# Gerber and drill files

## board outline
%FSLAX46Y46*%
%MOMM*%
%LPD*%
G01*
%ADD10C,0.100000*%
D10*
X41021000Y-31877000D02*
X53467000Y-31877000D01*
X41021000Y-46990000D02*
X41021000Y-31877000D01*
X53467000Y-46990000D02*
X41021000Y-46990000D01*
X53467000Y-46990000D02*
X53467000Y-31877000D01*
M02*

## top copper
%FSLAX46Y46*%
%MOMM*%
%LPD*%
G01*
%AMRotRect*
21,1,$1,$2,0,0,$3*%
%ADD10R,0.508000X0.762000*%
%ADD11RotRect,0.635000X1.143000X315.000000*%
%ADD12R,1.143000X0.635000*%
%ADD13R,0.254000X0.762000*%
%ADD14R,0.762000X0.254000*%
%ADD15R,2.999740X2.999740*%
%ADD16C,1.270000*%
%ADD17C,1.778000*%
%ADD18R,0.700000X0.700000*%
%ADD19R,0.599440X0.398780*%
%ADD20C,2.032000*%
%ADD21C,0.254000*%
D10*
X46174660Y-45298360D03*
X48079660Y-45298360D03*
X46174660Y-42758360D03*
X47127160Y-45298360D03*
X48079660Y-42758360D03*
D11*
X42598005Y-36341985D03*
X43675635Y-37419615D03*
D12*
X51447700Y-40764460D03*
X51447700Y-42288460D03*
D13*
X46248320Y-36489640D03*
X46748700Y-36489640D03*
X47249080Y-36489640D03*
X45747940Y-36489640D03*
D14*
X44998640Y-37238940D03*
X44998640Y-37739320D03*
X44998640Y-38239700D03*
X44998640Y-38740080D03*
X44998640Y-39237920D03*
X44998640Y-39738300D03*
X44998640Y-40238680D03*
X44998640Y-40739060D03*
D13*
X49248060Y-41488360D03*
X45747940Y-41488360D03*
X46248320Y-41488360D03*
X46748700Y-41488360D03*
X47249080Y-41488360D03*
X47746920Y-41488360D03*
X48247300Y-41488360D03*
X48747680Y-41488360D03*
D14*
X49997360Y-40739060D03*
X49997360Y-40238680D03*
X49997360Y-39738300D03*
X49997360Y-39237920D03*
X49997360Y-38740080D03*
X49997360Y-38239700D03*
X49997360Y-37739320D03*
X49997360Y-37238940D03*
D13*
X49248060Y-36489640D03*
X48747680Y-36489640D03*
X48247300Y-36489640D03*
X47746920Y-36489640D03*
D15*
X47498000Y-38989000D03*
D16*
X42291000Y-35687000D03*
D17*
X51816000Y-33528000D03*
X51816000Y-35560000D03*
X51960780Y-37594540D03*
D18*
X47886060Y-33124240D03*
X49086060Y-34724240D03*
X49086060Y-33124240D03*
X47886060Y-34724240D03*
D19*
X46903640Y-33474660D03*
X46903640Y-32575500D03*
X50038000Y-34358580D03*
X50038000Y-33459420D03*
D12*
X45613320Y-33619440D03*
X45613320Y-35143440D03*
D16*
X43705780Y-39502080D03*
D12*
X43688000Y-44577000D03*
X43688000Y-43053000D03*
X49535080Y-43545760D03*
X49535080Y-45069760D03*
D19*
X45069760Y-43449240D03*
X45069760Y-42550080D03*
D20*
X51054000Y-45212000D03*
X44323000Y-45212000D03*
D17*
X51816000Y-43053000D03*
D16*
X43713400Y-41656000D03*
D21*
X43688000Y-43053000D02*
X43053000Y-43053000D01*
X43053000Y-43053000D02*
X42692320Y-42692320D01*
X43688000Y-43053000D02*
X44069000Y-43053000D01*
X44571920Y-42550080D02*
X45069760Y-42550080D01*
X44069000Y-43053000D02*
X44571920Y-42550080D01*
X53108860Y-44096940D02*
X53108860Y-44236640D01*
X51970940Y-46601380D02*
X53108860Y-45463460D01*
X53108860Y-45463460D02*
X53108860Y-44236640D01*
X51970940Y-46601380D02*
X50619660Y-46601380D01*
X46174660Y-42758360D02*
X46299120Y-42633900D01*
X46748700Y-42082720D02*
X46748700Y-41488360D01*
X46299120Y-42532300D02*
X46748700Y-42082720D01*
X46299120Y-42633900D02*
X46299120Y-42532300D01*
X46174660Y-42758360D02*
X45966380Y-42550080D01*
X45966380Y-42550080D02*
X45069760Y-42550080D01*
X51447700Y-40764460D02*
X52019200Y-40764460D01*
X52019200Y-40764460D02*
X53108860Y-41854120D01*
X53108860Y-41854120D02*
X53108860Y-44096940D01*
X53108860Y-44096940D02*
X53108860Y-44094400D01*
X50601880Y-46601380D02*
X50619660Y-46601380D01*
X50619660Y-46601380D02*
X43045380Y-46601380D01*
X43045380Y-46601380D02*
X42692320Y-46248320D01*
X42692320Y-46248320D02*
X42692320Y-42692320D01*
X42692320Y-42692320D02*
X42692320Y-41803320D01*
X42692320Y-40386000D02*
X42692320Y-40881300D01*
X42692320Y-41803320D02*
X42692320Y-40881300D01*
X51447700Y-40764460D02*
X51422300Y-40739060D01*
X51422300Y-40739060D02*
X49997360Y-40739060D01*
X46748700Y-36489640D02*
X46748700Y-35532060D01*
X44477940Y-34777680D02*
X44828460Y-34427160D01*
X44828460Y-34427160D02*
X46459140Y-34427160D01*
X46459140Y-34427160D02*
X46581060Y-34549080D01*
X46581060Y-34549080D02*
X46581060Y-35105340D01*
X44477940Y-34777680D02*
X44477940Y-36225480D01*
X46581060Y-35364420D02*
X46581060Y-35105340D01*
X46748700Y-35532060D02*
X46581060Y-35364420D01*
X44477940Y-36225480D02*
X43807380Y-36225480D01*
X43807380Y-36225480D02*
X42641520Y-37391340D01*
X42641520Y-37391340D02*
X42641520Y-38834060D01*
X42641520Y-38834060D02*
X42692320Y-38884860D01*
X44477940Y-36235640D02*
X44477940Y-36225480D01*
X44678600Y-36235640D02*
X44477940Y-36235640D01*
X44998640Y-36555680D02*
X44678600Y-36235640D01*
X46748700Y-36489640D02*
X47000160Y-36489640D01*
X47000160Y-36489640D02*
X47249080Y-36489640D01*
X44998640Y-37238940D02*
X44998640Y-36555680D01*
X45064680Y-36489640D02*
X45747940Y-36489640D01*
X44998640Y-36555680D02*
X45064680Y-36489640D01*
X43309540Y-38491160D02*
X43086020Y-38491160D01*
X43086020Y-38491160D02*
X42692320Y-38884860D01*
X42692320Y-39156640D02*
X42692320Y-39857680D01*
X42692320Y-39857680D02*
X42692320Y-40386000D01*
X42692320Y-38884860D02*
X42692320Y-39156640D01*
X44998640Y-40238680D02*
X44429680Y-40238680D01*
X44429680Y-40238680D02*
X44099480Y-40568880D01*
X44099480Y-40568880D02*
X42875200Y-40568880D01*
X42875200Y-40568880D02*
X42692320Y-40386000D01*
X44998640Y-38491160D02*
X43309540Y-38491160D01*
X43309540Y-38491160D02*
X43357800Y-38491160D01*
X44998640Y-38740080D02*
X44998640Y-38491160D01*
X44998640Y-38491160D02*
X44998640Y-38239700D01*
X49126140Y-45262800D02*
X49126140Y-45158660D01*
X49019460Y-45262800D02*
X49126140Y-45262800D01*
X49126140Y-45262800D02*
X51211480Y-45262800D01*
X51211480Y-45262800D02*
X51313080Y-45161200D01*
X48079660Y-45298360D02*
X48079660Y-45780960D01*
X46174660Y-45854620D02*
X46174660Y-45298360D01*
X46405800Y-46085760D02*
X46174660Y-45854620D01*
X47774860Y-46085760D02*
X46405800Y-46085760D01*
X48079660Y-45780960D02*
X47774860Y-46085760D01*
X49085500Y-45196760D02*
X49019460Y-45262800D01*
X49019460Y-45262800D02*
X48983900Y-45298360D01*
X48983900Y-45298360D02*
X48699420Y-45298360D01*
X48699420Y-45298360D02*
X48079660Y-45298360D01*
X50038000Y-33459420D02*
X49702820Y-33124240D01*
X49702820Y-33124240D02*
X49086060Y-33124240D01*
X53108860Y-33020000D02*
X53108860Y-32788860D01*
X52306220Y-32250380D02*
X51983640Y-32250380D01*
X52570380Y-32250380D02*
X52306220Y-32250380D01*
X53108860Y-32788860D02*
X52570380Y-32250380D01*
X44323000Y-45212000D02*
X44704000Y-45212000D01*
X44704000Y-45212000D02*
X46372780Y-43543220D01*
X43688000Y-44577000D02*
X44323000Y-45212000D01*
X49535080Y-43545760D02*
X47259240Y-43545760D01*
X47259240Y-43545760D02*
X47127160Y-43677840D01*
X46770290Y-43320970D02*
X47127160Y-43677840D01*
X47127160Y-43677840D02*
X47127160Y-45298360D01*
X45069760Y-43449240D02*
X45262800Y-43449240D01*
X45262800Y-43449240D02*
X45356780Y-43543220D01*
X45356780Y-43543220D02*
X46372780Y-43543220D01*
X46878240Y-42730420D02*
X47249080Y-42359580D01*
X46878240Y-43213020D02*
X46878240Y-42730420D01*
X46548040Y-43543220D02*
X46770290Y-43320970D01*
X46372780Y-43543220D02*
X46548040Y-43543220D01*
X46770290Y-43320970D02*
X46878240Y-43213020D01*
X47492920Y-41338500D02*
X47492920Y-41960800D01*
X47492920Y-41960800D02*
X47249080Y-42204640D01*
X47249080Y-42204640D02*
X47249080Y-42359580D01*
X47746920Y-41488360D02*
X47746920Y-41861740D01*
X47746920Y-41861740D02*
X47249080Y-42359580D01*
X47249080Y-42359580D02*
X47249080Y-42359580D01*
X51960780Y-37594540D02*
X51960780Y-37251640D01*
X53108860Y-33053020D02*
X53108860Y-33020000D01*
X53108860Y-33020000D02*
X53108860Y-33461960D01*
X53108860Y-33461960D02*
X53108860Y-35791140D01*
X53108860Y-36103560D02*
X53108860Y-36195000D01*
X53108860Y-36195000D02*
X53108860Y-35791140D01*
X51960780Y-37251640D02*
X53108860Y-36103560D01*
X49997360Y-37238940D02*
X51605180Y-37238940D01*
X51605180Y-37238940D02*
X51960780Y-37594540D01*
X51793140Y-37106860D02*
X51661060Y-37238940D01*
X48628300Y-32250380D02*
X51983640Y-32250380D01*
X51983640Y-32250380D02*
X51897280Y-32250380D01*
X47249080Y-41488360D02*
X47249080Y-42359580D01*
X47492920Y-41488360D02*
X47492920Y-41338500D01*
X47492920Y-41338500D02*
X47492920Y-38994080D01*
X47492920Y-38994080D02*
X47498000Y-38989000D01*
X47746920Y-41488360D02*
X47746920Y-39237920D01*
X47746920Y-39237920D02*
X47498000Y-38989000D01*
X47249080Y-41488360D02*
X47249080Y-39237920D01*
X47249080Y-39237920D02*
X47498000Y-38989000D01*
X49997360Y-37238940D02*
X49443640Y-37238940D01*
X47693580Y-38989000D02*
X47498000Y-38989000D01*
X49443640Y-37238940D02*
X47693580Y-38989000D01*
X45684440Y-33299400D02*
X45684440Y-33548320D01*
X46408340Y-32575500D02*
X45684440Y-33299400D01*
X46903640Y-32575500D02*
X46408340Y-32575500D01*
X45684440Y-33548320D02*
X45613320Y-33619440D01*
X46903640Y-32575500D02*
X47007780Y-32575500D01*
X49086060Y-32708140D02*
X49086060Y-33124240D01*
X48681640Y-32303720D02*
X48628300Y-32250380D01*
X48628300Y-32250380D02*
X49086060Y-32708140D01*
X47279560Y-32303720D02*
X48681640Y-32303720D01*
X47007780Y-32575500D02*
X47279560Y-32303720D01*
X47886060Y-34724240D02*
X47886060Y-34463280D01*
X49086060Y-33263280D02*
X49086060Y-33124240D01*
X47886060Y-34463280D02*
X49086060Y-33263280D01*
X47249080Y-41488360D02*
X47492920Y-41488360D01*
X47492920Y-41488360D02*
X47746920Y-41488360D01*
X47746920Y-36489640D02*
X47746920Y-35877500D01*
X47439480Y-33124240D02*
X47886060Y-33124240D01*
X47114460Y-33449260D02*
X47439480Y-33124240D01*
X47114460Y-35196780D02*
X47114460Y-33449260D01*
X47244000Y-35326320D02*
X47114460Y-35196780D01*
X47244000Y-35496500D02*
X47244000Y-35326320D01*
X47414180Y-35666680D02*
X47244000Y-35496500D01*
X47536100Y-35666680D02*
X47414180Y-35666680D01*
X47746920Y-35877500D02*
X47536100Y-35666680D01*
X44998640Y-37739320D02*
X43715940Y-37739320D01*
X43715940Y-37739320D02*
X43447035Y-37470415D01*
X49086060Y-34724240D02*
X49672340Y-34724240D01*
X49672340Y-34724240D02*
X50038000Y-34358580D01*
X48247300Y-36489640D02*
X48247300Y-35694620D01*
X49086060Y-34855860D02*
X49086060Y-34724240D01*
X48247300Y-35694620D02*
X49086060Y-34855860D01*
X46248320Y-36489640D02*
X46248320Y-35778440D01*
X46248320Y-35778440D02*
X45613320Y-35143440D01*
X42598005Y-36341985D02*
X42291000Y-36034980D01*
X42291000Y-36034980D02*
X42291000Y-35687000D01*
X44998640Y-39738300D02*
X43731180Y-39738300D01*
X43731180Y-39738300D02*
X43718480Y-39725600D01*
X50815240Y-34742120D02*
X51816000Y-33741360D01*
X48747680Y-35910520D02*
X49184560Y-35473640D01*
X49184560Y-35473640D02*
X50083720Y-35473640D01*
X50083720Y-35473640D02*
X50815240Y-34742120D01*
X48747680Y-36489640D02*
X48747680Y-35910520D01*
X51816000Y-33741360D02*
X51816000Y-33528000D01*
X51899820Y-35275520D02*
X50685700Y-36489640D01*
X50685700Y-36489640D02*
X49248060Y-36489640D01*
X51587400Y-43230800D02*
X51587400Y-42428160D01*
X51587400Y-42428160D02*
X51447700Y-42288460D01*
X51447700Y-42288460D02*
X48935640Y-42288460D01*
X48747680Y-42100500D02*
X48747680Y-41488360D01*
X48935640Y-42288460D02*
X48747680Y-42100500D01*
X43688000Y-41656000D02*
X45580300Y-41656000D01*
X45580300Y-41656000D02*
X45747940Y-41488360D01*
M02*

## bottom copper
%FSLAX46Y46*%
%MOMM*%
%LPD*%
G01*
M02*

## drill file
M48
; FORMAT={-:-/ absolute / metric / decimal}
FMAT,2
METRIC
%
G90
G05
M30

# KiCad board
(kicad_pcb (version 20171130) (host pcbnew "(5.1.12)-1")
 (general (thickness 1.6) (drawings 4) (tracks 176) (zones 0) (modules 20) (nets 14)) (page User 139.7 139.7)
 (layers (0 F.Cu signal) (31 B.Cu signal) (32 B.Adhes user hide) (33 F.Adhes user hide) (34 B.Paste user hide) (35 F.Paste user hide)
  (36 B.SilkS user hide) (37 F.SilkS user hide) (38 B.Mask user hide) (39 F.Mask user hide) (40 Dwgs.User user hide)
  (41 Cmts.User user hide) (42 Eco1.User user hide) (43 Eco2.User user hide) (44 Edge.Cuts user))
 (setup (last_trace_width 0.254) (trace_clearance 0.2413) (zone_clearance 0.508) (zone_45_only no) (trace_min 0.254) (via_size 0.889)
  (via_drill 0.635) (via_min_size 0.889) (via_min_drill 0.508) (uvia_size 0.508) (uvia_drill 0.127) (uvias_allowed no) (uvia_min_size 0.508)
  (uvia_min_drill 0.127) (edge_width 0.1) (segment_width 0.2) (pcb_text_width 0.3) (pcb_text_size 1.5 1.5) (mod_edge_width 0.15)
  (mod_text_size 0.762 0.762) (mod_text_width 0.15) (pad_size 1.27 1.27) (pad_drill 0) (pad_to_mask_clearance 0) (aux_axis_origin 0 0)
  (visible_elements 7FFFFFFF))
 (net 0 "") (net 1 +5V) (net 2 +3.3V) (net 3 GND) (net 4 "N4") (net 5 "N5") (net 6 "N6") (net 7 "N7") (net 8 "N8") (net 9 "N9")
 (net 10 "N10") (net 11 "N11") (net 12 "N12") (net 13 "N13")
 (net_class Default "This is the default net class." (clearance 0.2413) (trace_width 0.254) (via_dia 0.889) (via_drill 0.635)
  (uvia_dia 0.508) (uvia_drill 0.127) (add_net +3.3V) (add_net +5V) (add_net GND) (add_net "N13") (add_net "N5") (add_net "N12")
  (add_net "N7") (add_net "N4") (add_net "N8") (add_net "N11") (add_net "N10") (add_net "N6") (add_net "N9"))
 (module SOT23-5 (layer F.Cu) (at 47.12716 44.02836)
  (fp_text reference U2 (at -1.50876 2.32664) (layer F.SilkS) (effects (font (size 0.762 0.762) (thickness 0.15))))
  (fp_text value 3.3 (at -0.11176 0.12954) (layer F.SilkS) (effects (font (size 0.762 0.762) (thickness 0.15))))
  (pad 1 smd rect (at -0.9525 1.27) (size 0.508 0.762) (layers F.Cu F.Paste F.Mask) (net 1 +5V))
  (pad 3 smd rect (at 0.9525 1.27) (size 0.508 0.762) (layers F.Cu F.Paste F.Mask) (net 1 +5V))
  (pad 5 smd rect (at -0.9525 -1.27) (size 0.508 0.762) (layers F.Cu F.Paste F.Mask) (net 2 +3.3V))
  (pad 2 smd rect (at 0 1.27) (size 0.508 0.762) (layers F.Cu F.Paste F.Mask) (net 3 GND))
  (pad 4 smd rect (at 0.9525 -1.27) (size 0.508 0.762) (layers F.Cu F.Paste F.Mask)))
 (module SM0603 (layer F.Cu) (at 43.13682 36.8808 315)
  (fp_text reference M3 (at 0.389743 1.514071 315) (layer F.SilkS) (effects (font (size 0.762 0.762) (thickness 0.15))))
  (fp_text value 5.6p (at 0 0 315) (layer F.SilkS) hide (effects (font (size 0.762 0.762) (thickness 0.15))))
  (pad 1 smd rect (at -0.762 0 315) (size 0.635 1.143) (layers F.Cu F.Paste F.Mask) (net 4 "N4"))
  (pad 2 smd rect (at 0.762 0 315) (size 0.635 1.143) (layers F.Cu F.Paste F.Mask) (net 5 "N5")))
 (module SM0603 (layer F.Cu) (at 51.4477 41.52646 270)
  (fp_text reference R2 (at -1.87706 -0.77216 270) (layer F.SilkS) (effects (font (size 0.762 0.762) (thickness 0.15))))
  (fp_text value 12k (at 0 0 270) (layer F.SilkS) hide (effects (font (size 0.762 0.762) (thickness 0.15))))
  (pad 1 smd rect (at -0.762 0 270) (size 0.635 1.143) (layers F.Cu F.Paste F.Mask) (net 2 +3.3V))
  (pad 2 smd rect (at 0.762 0 270) (size 0.635 1.143) (layers F.Cu F.Paste F.Mask) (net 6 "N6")))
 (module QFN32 (layer F.Cu) (at 47.498 38.989)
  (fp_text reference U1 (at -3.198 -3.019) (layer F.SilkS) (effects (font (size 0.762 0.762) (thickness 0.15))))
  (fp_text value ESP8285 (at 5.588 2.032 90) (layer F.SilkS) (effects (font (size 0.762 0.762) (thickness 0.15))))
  (pad 31 smd rect (at -1.24968 -2.49936) (size 0.254 0.762) (layers F.Cu F.Paste F.Mask) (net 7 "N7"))
  (pad 30 smd rect (at -0.7493 -2.49936) (size 0.254 0.762) (layers F.Cu F.Paste F.Mask) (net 2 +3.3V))
  (pad 29 smd rect (at -0.24892 -2.49936) (size 0.254 0.762) (layers F.Cu F.Paste F.Mask) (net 2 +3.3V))
  (pad 32 smd rect (at -1.75006 -2.49936) (size 0.254 0.762) (layers F.Cu F.Paste F.Mask) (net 2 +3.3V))
  (pad 1 smd rect (at -2.49936 -1.75006 90) (size 0.254 0.762) (layers F.Cu F.Paste F.Mask) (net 2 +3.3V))
  (pad 2 smd rect (at -2.49936 -1.24968 90) (size 0.254 0.762) (layers F.Cu F.Paste F.Mask) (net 5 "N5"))
  (pad 3 smd rect (at -2.49936 -0.7493 90) (size 0.254 0.762) (layers F.Cu F.Paste F.Mask) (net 2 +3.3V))
  (pad 4 smd rect (at -2.49936 -0.24892 90) (size 0.254 0.762) (layers F.Cu F.Paste F.Mask) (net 2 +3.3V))
  (pad 5 smd rect (at -2.49936 0.24892 90) (size 0.254 0.762) (layers F.Cu F.Paste F.Mask))
  (pad 6 smd rect (at -2.49936 0.7493 90) (size 0.254 0.762) (layers F.Cu F.Paste F.Mask) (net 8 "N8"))
  (pad 7 smd rect (at -2.49936 1.24968 90) (size 0.254 0.762) (layers F.Cu F.Paste F.Mask) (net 2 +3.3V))
  (pad 8 smd rect (at -2.49936 1.75006 90) (size 0.254 0.762) (layers F.Cu F.Paste F.Mask))
  (pad 16 smd rect (at 1.75006 2.49936) (size 0.254 0.762) (layers F.Cu F.Paste F.Mask))
  (pad 9 smd rect (at -1.75006 2.49936) (size 0.254 0.762) (layers F.Cu F.Paste F.Mask) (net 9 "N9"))
  (pad 10 smd rect (at -1.24968 2.49936) (size 0.254 0.762) (layers F.Cu F.Paste F.Mask))
  (pad 11 smd rect (at -0.7493 2.49936) (size 0.254 0.762) (layers F.Cu F.Paste F.Mask) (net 2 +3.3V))
  (pad 12 smd rect (at -0.24892 2.49936) (size 0.254 0.762) (layers F.Cu F.Paste F.Mask) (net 3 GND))
  (pad 13 smd rect (at 0.24892 2.49936) (size 0.254 0.762) (layers F.Cu F.Paste F.Mask) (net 3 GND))
  (pad 14 smd rect (at 0.7493 2.49936) (size 0.254 0.762) (layers F.Cu F.Paste F.Mask))
  (pad 15 smd rect (at 1.24968 2.49936) (size 0.254 0.762) (layers F.Cu F.Paste F.Mask) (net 6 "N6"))
  (pad 17 smd rect (at 2.49936 1.75006 90) (size 0.254 0.762) (layers F.Cu F.Paste F.Mask) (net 2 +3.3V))
  (pad 18 smd rect (at 2.49936 1.24968 90) (size 0.254 0.762) (layers F.Cu F.Paste F.Mask))
  (pad 19 smd rect (at 2.49936 0.7493 90) (size 0.254 0.762) (layers F.Cu F.Paste F.Mask))
  (pad 20 smd rect (at 2.49936 0.24892 90) (size 0.254 0.762) (layers F.Cu F.Paste F.Mask))
  (pad 21 smd rect (at 2.49936 -0.24892 90) (size 0.254 0.762) (layers F.Cu F.Paste F.Mask))
  (pad 22 smd rect (at 2.49936 -0.7493 90) (size 0.254 0.762) (layers F.Cu F.Paste F.Mask))
  (pad 23 smd rect (at 2.49936 -1.24968 90) (size 0.254 0.762) (layers F.Cu F.Paste F.Mask))
  (pad 24 smd rect (at 2.49936 -1.75006 90) (size 0.254 0.762) (layers F.Cu F.Paste F.Mask) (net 3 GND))
  (pad 25 smd rect (at 1.75006 -2.49936) (size 0.254 0.762) (layers F.Cu F.Paste F.Mask) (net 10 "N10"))
  (pad 26 smd rect (at 1.24968 -2.49936) (size 0.254 0.762) (layers F.Cu F.Paste F.Mask) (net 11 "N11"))
  (pad 27 smd rect (at 0.7493 -2.49936) (size 0.254 0.762) (layers F.Cu F.Paste F.Mask) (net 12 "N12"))
  (pad 28 smd rect (at 0.24892 -2.49936) (size 0.254 0.762) (layers F.Cu F.Paste F.Mask) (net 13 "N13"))
  (pad 33 smd rect (at 0 0) (size 2.99974 2.99974) (layers F.Cu F.Paste F.Mask) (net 3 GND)))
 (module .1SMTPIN (layer F.Cu) (at 42.291 35.687)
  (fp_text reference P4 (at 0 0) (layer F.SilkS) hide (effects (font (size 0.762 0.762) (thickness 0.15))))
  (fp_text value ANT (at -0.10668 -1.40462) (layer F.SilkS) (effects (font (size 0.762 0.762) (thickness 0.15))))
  (pad 1 smd circle (at 0 0) (size 1.27 1.27) (layers F.Cu F.Paste F.Mask) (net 4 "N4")))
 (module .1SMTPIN (layer F.Cu) (at 51.816 33.528)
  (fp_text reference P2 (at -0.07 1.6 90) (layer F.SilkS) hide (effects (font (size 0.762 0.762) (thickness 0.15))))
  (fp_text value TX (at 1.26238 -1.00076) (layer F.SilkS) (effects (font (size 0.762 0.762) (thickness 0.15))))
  (pad 1 smd circle (at 0 0) (size 1.778 1.778) (layers F.Cu F.Paste F.Mask) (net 11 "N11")))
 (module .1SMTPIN (layer F.Cu) (at 51.816 35.56)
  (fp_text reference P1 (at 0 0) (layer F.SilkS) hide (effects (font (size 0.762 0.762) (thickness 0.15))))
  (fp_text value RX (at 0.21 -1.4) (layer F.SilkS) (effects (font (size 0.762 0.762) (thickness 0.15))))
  (pad 1 smd circle (at 0 0) (size 1.778 1.778) (layers F.Cu F.Paste F.Mask) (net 10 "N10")))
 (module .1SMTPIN (layer F.Cu) (at 51.96078 37.59454)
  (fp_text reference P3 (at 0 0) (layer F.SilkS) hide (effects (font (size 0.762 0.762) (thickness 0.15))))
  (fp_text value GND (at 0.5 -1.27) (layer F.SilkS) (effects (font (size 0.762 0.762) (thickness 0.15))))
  (pad 1 smd circle (at 0 0) (size 1.778 1.778) (layers F.Cu F.Paste F.Mask) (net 3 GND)))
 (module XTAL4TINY (layer F.Cu) (at 48.48606 33.92424 270)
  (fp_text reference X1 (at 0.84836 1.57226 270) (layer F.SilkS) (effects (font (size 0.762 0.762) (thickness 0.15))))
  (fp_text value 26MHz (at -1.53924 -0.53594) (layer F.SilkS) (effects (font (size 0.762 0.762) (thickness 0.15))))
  (pad 1 smd rect (at -0.8 0.6 270) (size 0.7 0.7) (layers F.Cu F.Paste F.Mask) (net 13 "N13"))
  (pad 2 smd rect (at 0.8 -0.6 270) (size 0.7 0.7) (layers F.Cu F.Paste F.Mask) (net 12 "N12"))
  (pad 3 smd rect (at -0.8 -0.6 270) (size 0.7 0.7) (layers F.Cu F.Paste F.Mask) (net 3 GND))
  (pad 4 smd rect (at 0.8 0.6 270) (size 0.7 0.7) (layers F.Cu F.Paste F.Mask) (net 3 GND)))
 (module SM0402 (layer F.Cu) (at 46.90364 33.02508 90)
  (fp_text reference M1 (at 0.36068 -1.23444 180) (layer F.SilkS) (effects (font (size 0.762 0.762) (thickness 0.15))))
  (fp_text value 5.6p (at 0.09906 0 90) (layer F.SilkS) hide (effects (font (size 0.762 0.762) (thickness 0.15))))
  (pad 1 smd rect (at -0.44958 0 90) (size 0.39878 0.59944) (layers F.Cu F.Paste F.Mask) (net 13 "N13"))
  (pad 2 smd rect (at 0.44958 0 90) (size 0.39878 0.59944) (layers F.Cu F.Paste F.Mask) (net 3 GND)))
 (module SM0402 (layer F.Cu) (at 50.038 33.909 90)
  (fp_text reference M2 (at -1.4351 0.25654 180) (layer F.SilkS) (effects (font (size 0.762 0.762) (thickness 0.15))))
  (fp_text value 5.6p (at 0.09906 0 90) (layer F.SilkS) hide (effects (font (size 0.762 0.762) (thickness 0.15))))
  (pad 1 smd rect (at -0.44958 0 90) (size 0.39878 0.59944) (layers F.Cu F.Paste F.Mask) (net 12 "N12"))
  (pad 2 smd rect (at 0.44958 0 90) (size 0.39878 0.59944) (layers F.Cu F.Paste F.Mask) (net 3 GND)))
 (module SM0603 (layer F.Cu) (at 45.61332 34.38144 270)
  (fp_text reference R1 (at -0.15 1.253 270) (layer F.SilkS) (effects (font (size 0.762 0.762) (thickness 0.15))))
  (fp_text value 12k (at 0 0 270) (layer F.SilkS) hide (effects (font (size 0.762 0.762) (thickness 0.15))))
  (pad 1 smd rect (at -0.762 0 270) (size 0.635 1.143) (layers F.Cu F.Paste F.Mask) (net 3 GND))
  (pad 2 smd rect (at 0.762 0 270) (size 0.635 1.143) (layers F.Cu F.Paste F.Mask) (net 7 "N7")))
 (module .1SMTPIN (layer F.Cu) (at 43.70324 39.50208)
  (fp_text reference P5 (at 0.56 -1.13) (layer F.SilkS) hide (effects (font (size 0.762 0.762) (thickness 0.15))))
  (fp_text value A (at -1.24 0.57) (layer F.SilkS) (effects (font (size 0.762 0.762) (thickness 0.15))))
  (pad 1 smd circle (at 0.00254 0) (size 1.27 1.27) (layers F.Cu F.Paste F.Mask) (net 8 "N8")))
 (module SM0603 (layer F.Cu) (at 43.688 43.815 90)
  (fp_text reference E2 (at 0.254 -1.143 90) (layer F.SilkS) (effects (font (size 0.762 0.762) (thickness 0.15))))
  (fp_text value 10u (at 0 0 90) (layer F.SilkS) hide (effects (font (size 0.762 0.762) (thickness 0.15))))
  (pad 1 smd rect (at -0.762 0 90) (size 0.635 1.143) (layers F.Cu F.Paste F.Mask) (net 3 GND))
  (pad 2 smd rect (at 0.762 0 90) (size 0.635 1.143) (layers F.Cu F.Paste F.Mask) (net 2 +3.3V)))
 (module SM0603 (layer F.Cu) (at 49.53508 44.30776 270)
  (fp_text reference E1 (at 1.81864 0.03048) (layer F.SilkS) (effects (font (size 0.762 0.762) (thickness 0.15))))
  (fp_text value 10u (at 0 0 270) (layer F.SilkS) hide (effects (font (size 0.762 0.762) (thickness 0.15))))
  (pad 1 smd rect (at -0.762 0 270) (size 0.635 1.143) (layers F.Cu F.Paste F.Mask) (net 3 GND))
  (pad 2 smd rect (at 0.762 0 270) (size 0.635 1.143) (layers F.Cu F.Paste F.Mask) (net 1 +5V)))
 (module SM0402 (layer F.Cu) (at 45.06976 42.99966 90)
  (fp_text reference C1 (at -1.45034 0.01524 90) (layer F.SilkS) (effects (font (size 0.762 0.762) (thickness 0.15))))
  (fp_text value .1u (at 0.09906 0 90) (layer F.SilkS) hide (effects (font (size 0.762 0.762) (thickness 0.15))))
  (pad 1 smd rect (at -0.44958 0 90) (size 0.39878 0.59944) (layers F.Cu F.Paste F.Mask) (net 3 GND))
  (pad 2 smd rect (at 0.44958 0 90) (size 0.39878 0.59944) (layers F.Cu F.Paste F.Mask) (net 2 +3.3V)))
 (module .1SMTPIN (layer F.Cu) (at 51.054 45.212)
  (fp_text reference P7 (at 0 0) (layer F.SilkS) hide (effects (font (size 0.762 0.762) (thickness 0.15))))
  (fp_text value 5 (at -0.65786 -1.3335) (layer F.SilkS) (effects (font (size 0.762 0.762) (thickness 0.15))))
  (pad 1 smd circle (at 0 0) (size 2.032 2.032) (layers F.Cu F.Paste F.Mask) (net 1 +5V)))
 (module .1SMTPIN (layer F.Cu) (at 44.323 45.212)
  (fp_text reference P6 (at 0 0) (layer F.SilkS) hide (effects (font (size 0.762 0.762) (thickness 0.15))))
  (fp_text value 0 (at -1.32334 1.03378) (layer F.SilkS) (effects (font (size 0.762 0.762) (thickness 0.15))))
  (pad 1 smd circle (at 0 0) (size 2.032 2.032) (layers F.Cu F.Paste F.Mask) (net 3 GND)))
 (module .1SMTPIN (layer F.Cu) (at 51.816 43.053)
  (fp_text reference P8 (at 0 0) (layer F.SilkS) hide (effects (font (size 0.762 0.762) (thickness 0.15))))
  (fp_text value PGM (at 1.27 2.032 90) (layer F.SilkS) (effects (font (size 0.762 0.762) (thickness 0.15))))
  (pad 1 smd circle (at 0 0) (size 1.778 1.778) (layers F.Cu F.Paste F.Mask) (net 6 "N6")))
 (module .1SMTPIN (layer F.Cu) (at 43.688 41.656)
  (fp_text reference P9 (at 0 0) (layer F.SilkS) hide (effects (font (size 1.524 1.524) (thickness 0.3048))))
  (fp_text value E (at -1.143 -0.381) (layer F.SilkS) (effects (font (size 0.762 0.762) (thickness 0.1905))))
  (pad 1 smd circle (at 0.0254 0) (size 1.27 1.27) (layers F.Cu F.Paste F.Mask) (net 9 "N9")))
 (gr_line (start 41.021 31.877) (end 53.467 31.877) (angle 90) (layer Edge.Cuts) (width 0.1))
 (gr_line (start 41.021 46.99) (end 41.021 31.877) (angle 90) (layer Edge.Cuts) (width 0.1))
 (gr_line (start 53.467 46.99) (end 41.021 46.99) (angle 90) (layer Edge.Cuts) (width 0.1))
 (gr_line (start 53.467 46.99) (end 53.467 31.877) (angle 90) (layer Edge.Cuts) (width 0.1))
 (segment (start 43.688 43.053) (end 43.053 43.053) (width 0.254) (layer F.Cu) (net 2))
 (segment (start 43.053 43.053) (end 42.69232 42.69232) (width 0.254) (layer F.Cu) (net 2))
 (segment (start 43.688 43.053) (end 44.069 43.053) (width 0.254) (layer F.Cu) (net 2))
 (segment (start 44.57192 42.55008) (end 45.06976 42.55008) (width 0.254) (layer F.Cu) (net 2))
 (segment (start 44.069 43.053) (end 44.57192 42.55008) (width 0.254) (layer F.Cu) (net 2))
 (segment (start 53.10886 44.09694) (end 53.10886 44.23664) (width 0.254) (layer F.Cu) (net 2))
 (segment (start 51.97094 46.60138) (end 53.10886 45.46346) (width 0.254) (layer F.Cu) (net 2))
 (segment (start 53.10886 45.46346) (end 53.10886 44.23664) (width 0.254) (layer F.Cu) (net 2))
 (segment (start 51.97094 46.60138) (end 50.61966 46.60138) (width 0.254) (layer F.Cu) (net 2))
 (segment (start 46.17466 42.75836) (end 46.29912 42.6339) (width 0.254) (layer F.Cu) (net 2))
 (segment (start 46.7487 42.08272) (end 46.7487 41.48836) (width 0.254) (layer F.Cu) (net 2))
 (segment (start 46.29912 42.5323) (end 46.7487 42.08272) (width 0.254) (layer F.Cu) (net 2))
 (segment (start 46.29912 42.6339) (end 46.29912 42.5323) (width 0.254) (layer F.Cu) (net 2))
 (segment (start 46.17466 42.75836) (end 45.96638 42.55008) (width 0.254) (layer F.Cu) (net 2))
 (segment (start 45.96638 42.55008) (end 45.06976 42.55008) (width 0.254) (layer F.Cu) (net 2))
 (segment (start 51.4477 40.76446) (end 52.0192 40.76446) (width 0.254) (layer F.Cu) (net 2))
 (segment (start 52.0192 40.76446) (end 53.10886 41.85412) (width 0.254) (layer F.Cu) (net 2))
 (segment (start 53.10886 41.85412) (end 53.10886 44.09694) (width 0.254) (layer F.Cu) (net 2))
 (segment (start 53.10886 44.09694) (end 53.10886 44.0944) (width 0.254) (layer F.Cu) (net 2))
 (segment (start 50.60188 46.60138) (end 50.61966 46.60138) (width 0.254) (layer F.Cu) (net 2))
 (segment (start 50.61966 46.60138) (end 43.04538 46.60138) (width 0.254) (layer F.Cu) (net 2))
 (segment (start 43.04538 46.60138) (end 42.69232 46.24832) (width 0.254) (layer F.Cu) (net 2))
 (segment (start 42.69232 46.24832) (end 42.69232 42.69232) (width 0.254) (layer F.Cu) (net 2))
 (segment (start 42.69232 42.69232) (end 42.69232 41.80332) (width 0.254) (layer F.Cu) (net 2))
 (segment (start 42.69232 40.386) (end 42.69232 40.8813) (width 0.254) (layer F.Cu) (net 2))
 (segment (start 42.69232 41.80332) (end 42.69232 40.8813) (width 0.254) (layer F.Cu) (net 2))
 (segment (start 51.4477 40.76446) (end 51.4223 40.73906) (width 0.254) (layer F.Cu) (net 2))
 (segment (start 51.4223 40.73906) (end 49.99736 40.73906) (width 0.254) (layer F.Cu) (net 2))
 (segment (start 46.7487 36.48964) (end 46.7487 35.53206) (width 0.254) (layer F.Cu) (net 2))
 (segment (start 44.47794 34.77768) (end 44.82846 34.42716) (width 0.254) (layer F.Cu) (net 2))
 (segment (start 44.82846 34.42716) (end 46.45914 34.42716) (width 0.254) (layer F.Cu) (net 2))
 (segment (start 46.45914 34.42716) (end 46.58106 34.54908) (width 0.254) (layer F.Cu) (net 2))
 (segment (start 46.58106 34.54908) (end 46.58106 35.10534) (width 0.254) (layer F.Cu) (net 2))
 (segment (start 44.47794 34.77768) (end 44.47794 36.22548) (width 0.254) (layer F.Cu) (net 2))
 (segment (start 46.58106 35.36442) (end 46.58106 35.10534) (width 0.254) (layer F.Cu) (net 2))
 (segment (start 46.7487 35.53206) (end 46.58106 35.36442) (width 0.254) (layer F.Cu) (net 2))
 (segment (start 44.47794 36.22548) (end 43.80738 36.22548) (width 0.254) (layer F.Cu) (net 2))
 (segment (start 43.80738 36.22548) (end 42.64152 37.39134) (width 0.254) (layer F.Cu) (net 2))
 (segment (start 42.64152 37.39134) (end 42.64152 38.83406) (width 0.254) (layer F.Cu) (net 2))
 (segment (start 42.64152 38.83406) (end 42.69232 38.88486) (width 0.254) (layer F.Cu) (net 2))
 (segment (start 44.47794 36.23564) (end 44.47794 36.22548) (width 0.254) (layer F.Cu) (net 2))
 (segment (start 44.6786 36.23564) (end 44.47794 36.23564) (width 0.254) (layer F.Cu) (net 2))
 (segment (start 44.99864 36.55568) (end 44.6786 36.23564) (width 0.254) (layer F.Cu) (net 2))
 (segment (start 46.7487 36.48964) (end 47.00016 36.48964) (width 0.254) (layer F.Cu) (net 2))
 (segment (start 47.00016 36.48964) (end 47.24908 36.48964) (width 0.254) (layer F.Cu) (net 2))
 (segment (start 44.99864 37.23894) (end 44.99864 36.55568) (width 0.254) (layer F.Cu) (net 2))
 (segment (start 45.06468 36.48964) (end 45.74794 36.48964) (width 0.254) (layer F.Cu) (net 2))
 (segment (start 44.99864 36.55568) (end 45.06468 36.48964) (width 0.254) (layer F.Cu) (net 2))
 (segment (start 43.30954 38.49116) (end 43.08602 38.49116) (width 0.254) (layer F.Cu) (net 2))
 (segment (start 43.08602 38.49116) (end 42.69232 38.88486) (width 0.254) (layer F.Cu) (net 2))
 (segment (start 42.69232 39.15664) (end 42.69232 39.85768) (width 0.254) (layer F.Cu) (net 2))
 (segment (start 42.69232 39.85768) (end 42.69232 40.386) (width 0.254) (layer F.Cu) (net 2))
 (segment (start 42.69232 38.88486) (end 42.69232 39.15664) (width 0.254) (layer F.Cu) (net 2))
 (segment (start 44.99864 40.23868) (end 44.42968 40.23868) (width 0.254) (layer F.Cu) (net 2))
 (segment (start 44.42968 40.23868) (end 44.09948 40.56888) (width 0.254) (layer F.Cu) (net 2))
 (segment (start 44.09948 40.56888) (end 42.8752 40.56888) (width 0.254) (layer F.Cu) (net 2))
 (segment (start 42.8752 40.56888) (end 42.69232 40.386) (width 0.254) (layer F.Cu) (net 2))
 (segment (start 44.99864 38.49116) (end 43.30954 38.49116) (width 0.254) (layer F.Cu) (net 2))
 (segment (start 43.30954 38.49116) (end 43.3578 38.49116) (width 0.254) (layer F.Cu) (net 2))
 (segment (start 44.99864 38.74008) (end 44.99864 38.49116) (width 0.254) (layer F.Cu) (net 2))
 (segment (start 44.99864 38.49116) (end 44.99864 38.2397) (width 0.254) (layer F.Cu) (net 2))
 (segment (start 49.12614 45.2628) (end 49.12614 45.15866) (width 0.254) (layer F.Cu) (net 1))
 (segment (start 49.01946 45.2628) (end 49.12614 45.2628) (width 0.254) (layer F.Cu) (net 1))
 (segment (start 49.12614 45.2628) (end 51.21148 45.2628) (width 0.254) (layer F.Cu) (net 1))
 (segment (start 51.21148 45.2628) (end 51.31308 45.1612) (width 0.254) (layer F.Cu) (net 1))
 (segment (start 48.07966 45.29836) (end 48.07966 45.78096) (width 0.254) (layer F.Cu) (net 1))
 (segment (start 46.17466 45.85462) (end 46.17466 45.29836) (width 0.254) (layer F.Cu) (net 1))
 (segment (start 46.4058 46.08576) (end 46.17466 45.85462) (width 0.254) (layer F.Cu) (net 1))
 (segment (start 47.77486 46.08576) (end 46.4058 46.08576) (width 0.254) (layer F.Cu) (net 1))
 (segment (start 48.07966 45.78096) (end 47.77486 46.08576) (width 0.254) (layer F.Cu) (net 1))
 (segment (start 49.0855 45.19676) (end 49.01946 45.2628) (width 0.254) (layer F.Cu) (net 1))
 (segment (start 49.01946 45.2628) (end 48.9839 45.29836) (width 0.254) (layer F.Cu) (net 1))
 (segment (start 48.9839 45.29836) (end 48.69942 45.29836) (width 0.254) (layer F.Cu) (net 1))
 (segment (start 48.69942 45.29836) (end 48.07966 45.29836) (width 0.254) (layer F.Cu) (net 1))
 (segment (start 50.038 33.45942) (end 49.70282 33.12424) (width 0.254) (layer F.Cu) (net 3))
 (segment (start 49.70282 33.12424) (end 49.08606 33.12424) (width 0.254) (layer F.Cu) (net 3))
 (segment (start 53.10886 33.02) (end 53.10886 32.78886) (width 0.254) (layer F.Cu) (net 3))
 (segment (start 52.30622 32.25038) (end 51.98364 32.25038) (width 0.254) (layer F.Cu) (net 3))
 (segment (start 52.57038 32.25038) (end 52.30622 32.25038) (width 0.254) (layer F.Cu) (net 3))
 (segment (start 53.10886 32.78886) (end 52.57038 32.25038) (width 0.254) (layer F.Cu) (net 3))
 (segment (start 44.323 45.212) (end 44.704 45.212) (width 0.254) (layer F.Cu) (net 3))
 (segment (start 44.704 45.212) (end 46.37278 43.54322) (width 0.254) (layer F.Cu) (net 3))
 (segment (start 43.688 44.577) (end 44.323 45.212) (width 0.254) (layer F.Cu) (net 3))
 (segment (start 49.53508 43.54576) (end 47.25924 43.54576) (width 0.254) (layer F.Cu) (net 3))
 (segment (start 47.25924 43.54576) (end 47.12716 43.67784) (width 0.254) (layer F.Cu) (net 3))
 (segment (start 46.77029 43.32097) (end 47.12716 43.67784) (width 0.254) (layer F.Cu) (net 3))
 (segment (start 47.12716 43.67784) (end 47.12716 45.29836) (width 0.254) (layer F.Cu) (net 3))
 (segment (start 45.06976 43.44924) (end 45.2628 43.44924) (width 0.254) (layer F.Cu) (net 3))
 (segment (start 45.2628 43.44924) (end 45.35678 43.54322) (width 0.254) (layer F.Cu) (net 3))
 (segment (start 45.35678 43.54322) (end 46.37278 43.54322) (width 0.254) (layer F.Cu) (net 3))
 (segment (start 46.87824 42.73042) (end 47.24908 42.35958) (width 0.254) (layer F.Cu) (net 3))
 (segment (start 46.87824 43.21302) (end 46.87824 42.73042) (width 0.254) (layer F.Cu) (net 3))
 (segment (start 46.54804 43.54322) (end 46.77029 43.32097) (width 0.254) (layer F.Cu) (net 3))
 (segment (start 46.37278 43.54322) (end 46.54804 43.54322) (width 0.254) (layer F.Cu) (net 3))
 (segment (start 46.77029 43.32097) (end 46.87824 43.21302) (width 0.254) (layer F.Cu) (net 3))
 (segment (start 47.49292 41.3385) (end 47.49292 41.9608) (width 0.254) (layer F.Cu) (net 3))
 (segment (start 47.49292 41.9608) (end 47.24908 42.20464) (width 0.254) (layer F.Cu) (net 3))
 (segment (start 47.24908 42.20464) (end 47.24908 42.35958) (width 0.254) (layer F.Cu) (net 3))
 (segment (start 47.74692 41.48836) (end 47.74692 41.86174) (width 0.254) (layer F.Cu) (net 3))
 (segment (start 47.74692 41.86174) (end 47.24908 42.35958) (width 0.254) (layer F.Cu) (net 3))
 (segment (start 47.24908 42.35958) (end 47.24908 42.35958) (width 0.254) (layer F.Cu) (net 3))
 (segment (start 51.96078 37.59454) (end 51.96078 37.25164) (width 0.254) (layer F.Cu) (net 3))
 (segment (start 53.10886 33.05302) (end 53.10886 33.02) (width 0.254) (layer F.Cu) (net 3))
 (segment (start 53.10886 33.02) (end 53.10886 33.46196) (width 0.254) (layer F.Cu) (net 3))
 (segment (start 53.10886 33.46196) (end 53.10886 35.79114) (width 0.254) (layer F.Cu) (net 3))
 (segment (start 53.10886 36.10356) (end 53.10886 36.195) (width 0.254) (layer F.Cu) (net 3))
 (segment (start 53.10886 36.195) (end 53.10886 35.79114) (width 0.254) (layer F.Cu) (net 3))
 (segment (start 51.96078 37.25164) (end 53.10886 36.10356) (width 0.254) (layer F.Cu) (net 3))
 (segment (start 49.99736 37.23894) (end 51.60518 37.23894) (width 0.254) (layer F.Cu) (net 3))
 (segment (start 51.60518 37.23894) (end 51.96078 37.59454) (width 0.254) (layer F.Cu) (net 3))
 (segment (start 51.79314 37.10686) (end 51.66106 37.23894) (width 0.254) (layer F.Cu) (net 3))
 (segment (start 48.6283 32.25038) (end 51.98364 32.25038) (width 0.254) (layer F.Cu) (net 3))
 (segment (start 51.98364 32.25038) (end 51.89728 32.25038) (width 0.254) (layer F.Cu) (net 3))
 (segment (start 47.24908 41.48836) (end 47.24908 42.35958) (width 0.254) (layer F.Cu) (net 3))
 (segment (start 47.49292 41.48836) (end 47.49292 41.3385) (width 0.254) (layer F.Cu) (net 3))
 (segment (start 47.49292 41.3385) (end 47.49292 38.99408) (width 0.254) (layer F.Cu) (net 3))
 (segment (start 47.49292 38.99408) (end 47.498 38.989) (width 0.254) (layer F.Cu) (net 3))
 (segment (start 47.74692 41.48836) (end 47.74692 39.23792) (width 0.254) (layer F.Cu) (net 3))
 (segment (start 47.74692 39.23792) (end 47.498 38.989) (width 0.254) (layer F.Cu) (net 3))
 (segment (start 47.24908 41.48836) (end 47.24908 39.23792) (width 0.254) (layer F.Cu) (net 3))
 (segment (start 47.24908 39.23792) (end 47.498 38.989) (width 0.254) (layer F.Cu) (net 3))
 (segment (start 49.99736 37.23894) (end 49.44364 37.23894) (width 0.254) (layer F.Cu) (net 3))
 (segment (start 47.69358 38.989) (end 47.498 38.989) (width 0.254) (layer F.Cu) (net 3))
 (segment (start 49.44364 37.23894) (end 47.69358 38.989) (width 0.254) (layer F.Cu) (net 3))
 (segment (start 45.68444 33.2994) (end 45.68444 33.54832) (width 0.254) (layer F.Cu) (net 3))
 (segment (start 46.40834 32.5755) (end 45.68444 33.2994) (width 0.254) (layer F.Cu) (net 3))
 (segment (start 46.90364 32.5755) (end 46.40834 32.5755) (width 0.254) (layer F.Cu) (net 3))
 (segment (start 45.68444 33.54832) (end 45.61332 33.61944) (width 0.254) (layer F.Cu) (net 3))
 (segment (start 46.90364 32.5755) (end 47.00778 32.5755) (width 0.254) (layer F.Cu) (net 3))
 (segment (start 49.08606 32.70814) (end 49.08606 33.12424) (width 0.254) (layer F.Cu) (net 3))
 (segment (start 48.68164 32.30372) (end 48.6283 32.25038) (width 0.254) (layer F.Cu) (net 3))
 (segment (start 48.6283 32.25038) (end 49.08606 32.70814) (width 0.254) (layer F.Cu) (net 3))
 (segment (start 47.27956 32.30372) (end 48.68164 32.30372) (width 0.254) (layer F.Cu) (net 3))
 (segment (start 47.00778 32.5755) (end 47.27956 32.30372) (width 0.254) (layer F.Cu) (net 3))
 (segment (start 47.88606 34.72424) (end 47.88606 34.46328) (width 0.254) (layer F.Cu) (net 3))
 (segment (start 49.08606 33.26328) (end 49.08606 33.12424) (width 0.254) (layer F.Cu) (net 3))
 (segment (start 47.88606 34.46328) (end 49.08606 33.26328) (width 0.254) (layer F.Cu) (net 3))
 (segment (start 47.24908 41.48836) (end 47.49292 41.48836) (width 0.254) (layer F.Cu) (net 3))
 (segment (start 47.49292 41.48836) (end 47.74692 41.48836) (width 0.254) (layer F.Cu) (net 3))
 (segment (start 47.74692 36.48964) (end 47.74692 35.8775) (width 0.254) (layer F.Cu) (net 13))
 (segment (start 47.43948 33.12424) (end 47.88606 33.12424) (width 0.254) (layer F.Cu) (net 13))
 (segment (start 47.11446 33.44926) (end 47.43948 33.12424) (width 0.254) (layer F.Cu) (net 13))
 (segment (start 47.11446 35.19678) (end 47.11446 33.44926) (width 0.254) (layer F.Cu) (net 13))
 (segment (start 47.244 35.32632) (end 47.11446 35.19678) (width 0.254) (layer F.Cu) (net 13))
 (segment (start 47.244 35.4965) (end 47.244 35.32632) (width 0.254) (layer F.Cu) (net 13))
 (segment (start 47.41418 35.66668) (end 47.244 35.4965) (width 0.254) (layer F.Cu) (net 13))
 (segment (start 47.5361 35.66668) (end 47.41418 35.66668) (width 0.254) (layer F.Cu) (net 13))
 (segment (start 47.74692 35.8775) (end 47.5361 35.66668) (width 0.254) (layer F.Cu) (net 13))
 (segment (start 44.99864 37.73932) (end 43.71594 37.73932) (width 0.254) (layer F.Cu) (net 5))
 (segment (start 43.71594 37.73932) (end 43.447035 37.470415) (width 0.254) (layer F.Cu) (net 5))
 (segment (start 49.08606 34.72424) (end 49.67234 34.72424) (width 0.254) (layer F.Cu) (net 12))
 (segment (start 49.67234 34.72424) (end 50.038 34.35858) (width 0.254) (layer F.Cu) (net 12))
 (segment (start 48.2473 36.48964) (end 48.2473 35.69462) (width 0.254) (layer F.Cu) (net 12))
 (segment (start 49.08606 34.85586) (end 49.08606 34.72424) (width 0.254) (layer F.Cu) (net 12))
 (segment (start 48.2473 35.69462) (end 49.08606 34.85586) (width 0.254) (layer F.Cu) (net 12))
 (segment (start 46.24832 36.48964) (end 46.24832 35.77844) (width 0.254) (layer F.Cu) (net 7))
 (segment (start 46.24832 35.77844) (end 45.61332 35.14344) (width 0.254) (layer F.Cu) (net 7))
 (segment (start 42.598005 36.341985) (end 42.291 36.03498) (width 0.254) (layer F.Cu) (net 4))
 (segment (start 42.291 36.03498) (end 42.291 35.687) (width 0.254) (layer F.Cu) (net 4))
 (segment (start 44.99864 39.7383) (end 43.73118 39.7383) (width 0.254) (layer F.Cu) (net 8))
 (segment (start 43.73118 39.7383) (end 43.71848 39.7256) (width 0.254) (layer F.Cu) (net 8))
 (segment (start 50.81524 34.74212) (end 51.816 33.74136) (width 0.254) (layer F.Cu) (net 11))
 (segment (start 48.74768 35.91052) (end 49.18456 35.47364) (width 0.254) (layer F.Cu) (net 11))
 (segment (start 49.18456 35.47364) (end 50.08372 35.47364) (width 0.254) (layer F.Cu) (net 11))
 (segment (start 50.08372 35.47364) (end 50.81524 34.74212) (width 0.254) (layer F.Cu) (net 11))
 (segment (start 48.74768 36.48964) (end 48.74768 35.91052) (width 0.254) (layer F.Cu) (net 11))
 (segment (start 51.816 33.74136) (end 51.816 33.528) (width 0.254) (layer F.Cu) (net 11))
 (segment (start 51.89982 35.27552) (end 50.6857 36.48964) (width 0.254) (layer F.Cu) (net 10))
 (segment (start 50.6857 36.48964) (end 49.24806 36.48964) (width 0.254) (layer F.Cu) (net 10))
 (segment (start 51.5874 43.2308) (end 51.5874 42.42816) (width 0.254) (layer F.Cu) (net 6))
 (segment (start 51.5874 42.42816) (end 51.4477 42.28846) (width 0.254) (layer F.Cu) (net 6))
 (segment (start 51.4477 42.28846) (end 48.93564 42.28846) (width 0.254) (layer F.Cu) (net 6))
 (segment (start 48.74768 42.1005) (end 48.74768 41.48836) (width 0.254) (layer F.Cu) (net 6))
 (segment (start 48.93564 42.28846) (end 48.74768 42.1005) (width 0.254) (layer F.Cu) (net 6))
 (segment (start 43.688 41.656) (end 45.5803 41.656) (width 0.254) (layer F.Cu) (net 9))
 (segment (start 45.5803 41.656) (end 45.74794 41.48836) (width 0.254) (layer F.Cu) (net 9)))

